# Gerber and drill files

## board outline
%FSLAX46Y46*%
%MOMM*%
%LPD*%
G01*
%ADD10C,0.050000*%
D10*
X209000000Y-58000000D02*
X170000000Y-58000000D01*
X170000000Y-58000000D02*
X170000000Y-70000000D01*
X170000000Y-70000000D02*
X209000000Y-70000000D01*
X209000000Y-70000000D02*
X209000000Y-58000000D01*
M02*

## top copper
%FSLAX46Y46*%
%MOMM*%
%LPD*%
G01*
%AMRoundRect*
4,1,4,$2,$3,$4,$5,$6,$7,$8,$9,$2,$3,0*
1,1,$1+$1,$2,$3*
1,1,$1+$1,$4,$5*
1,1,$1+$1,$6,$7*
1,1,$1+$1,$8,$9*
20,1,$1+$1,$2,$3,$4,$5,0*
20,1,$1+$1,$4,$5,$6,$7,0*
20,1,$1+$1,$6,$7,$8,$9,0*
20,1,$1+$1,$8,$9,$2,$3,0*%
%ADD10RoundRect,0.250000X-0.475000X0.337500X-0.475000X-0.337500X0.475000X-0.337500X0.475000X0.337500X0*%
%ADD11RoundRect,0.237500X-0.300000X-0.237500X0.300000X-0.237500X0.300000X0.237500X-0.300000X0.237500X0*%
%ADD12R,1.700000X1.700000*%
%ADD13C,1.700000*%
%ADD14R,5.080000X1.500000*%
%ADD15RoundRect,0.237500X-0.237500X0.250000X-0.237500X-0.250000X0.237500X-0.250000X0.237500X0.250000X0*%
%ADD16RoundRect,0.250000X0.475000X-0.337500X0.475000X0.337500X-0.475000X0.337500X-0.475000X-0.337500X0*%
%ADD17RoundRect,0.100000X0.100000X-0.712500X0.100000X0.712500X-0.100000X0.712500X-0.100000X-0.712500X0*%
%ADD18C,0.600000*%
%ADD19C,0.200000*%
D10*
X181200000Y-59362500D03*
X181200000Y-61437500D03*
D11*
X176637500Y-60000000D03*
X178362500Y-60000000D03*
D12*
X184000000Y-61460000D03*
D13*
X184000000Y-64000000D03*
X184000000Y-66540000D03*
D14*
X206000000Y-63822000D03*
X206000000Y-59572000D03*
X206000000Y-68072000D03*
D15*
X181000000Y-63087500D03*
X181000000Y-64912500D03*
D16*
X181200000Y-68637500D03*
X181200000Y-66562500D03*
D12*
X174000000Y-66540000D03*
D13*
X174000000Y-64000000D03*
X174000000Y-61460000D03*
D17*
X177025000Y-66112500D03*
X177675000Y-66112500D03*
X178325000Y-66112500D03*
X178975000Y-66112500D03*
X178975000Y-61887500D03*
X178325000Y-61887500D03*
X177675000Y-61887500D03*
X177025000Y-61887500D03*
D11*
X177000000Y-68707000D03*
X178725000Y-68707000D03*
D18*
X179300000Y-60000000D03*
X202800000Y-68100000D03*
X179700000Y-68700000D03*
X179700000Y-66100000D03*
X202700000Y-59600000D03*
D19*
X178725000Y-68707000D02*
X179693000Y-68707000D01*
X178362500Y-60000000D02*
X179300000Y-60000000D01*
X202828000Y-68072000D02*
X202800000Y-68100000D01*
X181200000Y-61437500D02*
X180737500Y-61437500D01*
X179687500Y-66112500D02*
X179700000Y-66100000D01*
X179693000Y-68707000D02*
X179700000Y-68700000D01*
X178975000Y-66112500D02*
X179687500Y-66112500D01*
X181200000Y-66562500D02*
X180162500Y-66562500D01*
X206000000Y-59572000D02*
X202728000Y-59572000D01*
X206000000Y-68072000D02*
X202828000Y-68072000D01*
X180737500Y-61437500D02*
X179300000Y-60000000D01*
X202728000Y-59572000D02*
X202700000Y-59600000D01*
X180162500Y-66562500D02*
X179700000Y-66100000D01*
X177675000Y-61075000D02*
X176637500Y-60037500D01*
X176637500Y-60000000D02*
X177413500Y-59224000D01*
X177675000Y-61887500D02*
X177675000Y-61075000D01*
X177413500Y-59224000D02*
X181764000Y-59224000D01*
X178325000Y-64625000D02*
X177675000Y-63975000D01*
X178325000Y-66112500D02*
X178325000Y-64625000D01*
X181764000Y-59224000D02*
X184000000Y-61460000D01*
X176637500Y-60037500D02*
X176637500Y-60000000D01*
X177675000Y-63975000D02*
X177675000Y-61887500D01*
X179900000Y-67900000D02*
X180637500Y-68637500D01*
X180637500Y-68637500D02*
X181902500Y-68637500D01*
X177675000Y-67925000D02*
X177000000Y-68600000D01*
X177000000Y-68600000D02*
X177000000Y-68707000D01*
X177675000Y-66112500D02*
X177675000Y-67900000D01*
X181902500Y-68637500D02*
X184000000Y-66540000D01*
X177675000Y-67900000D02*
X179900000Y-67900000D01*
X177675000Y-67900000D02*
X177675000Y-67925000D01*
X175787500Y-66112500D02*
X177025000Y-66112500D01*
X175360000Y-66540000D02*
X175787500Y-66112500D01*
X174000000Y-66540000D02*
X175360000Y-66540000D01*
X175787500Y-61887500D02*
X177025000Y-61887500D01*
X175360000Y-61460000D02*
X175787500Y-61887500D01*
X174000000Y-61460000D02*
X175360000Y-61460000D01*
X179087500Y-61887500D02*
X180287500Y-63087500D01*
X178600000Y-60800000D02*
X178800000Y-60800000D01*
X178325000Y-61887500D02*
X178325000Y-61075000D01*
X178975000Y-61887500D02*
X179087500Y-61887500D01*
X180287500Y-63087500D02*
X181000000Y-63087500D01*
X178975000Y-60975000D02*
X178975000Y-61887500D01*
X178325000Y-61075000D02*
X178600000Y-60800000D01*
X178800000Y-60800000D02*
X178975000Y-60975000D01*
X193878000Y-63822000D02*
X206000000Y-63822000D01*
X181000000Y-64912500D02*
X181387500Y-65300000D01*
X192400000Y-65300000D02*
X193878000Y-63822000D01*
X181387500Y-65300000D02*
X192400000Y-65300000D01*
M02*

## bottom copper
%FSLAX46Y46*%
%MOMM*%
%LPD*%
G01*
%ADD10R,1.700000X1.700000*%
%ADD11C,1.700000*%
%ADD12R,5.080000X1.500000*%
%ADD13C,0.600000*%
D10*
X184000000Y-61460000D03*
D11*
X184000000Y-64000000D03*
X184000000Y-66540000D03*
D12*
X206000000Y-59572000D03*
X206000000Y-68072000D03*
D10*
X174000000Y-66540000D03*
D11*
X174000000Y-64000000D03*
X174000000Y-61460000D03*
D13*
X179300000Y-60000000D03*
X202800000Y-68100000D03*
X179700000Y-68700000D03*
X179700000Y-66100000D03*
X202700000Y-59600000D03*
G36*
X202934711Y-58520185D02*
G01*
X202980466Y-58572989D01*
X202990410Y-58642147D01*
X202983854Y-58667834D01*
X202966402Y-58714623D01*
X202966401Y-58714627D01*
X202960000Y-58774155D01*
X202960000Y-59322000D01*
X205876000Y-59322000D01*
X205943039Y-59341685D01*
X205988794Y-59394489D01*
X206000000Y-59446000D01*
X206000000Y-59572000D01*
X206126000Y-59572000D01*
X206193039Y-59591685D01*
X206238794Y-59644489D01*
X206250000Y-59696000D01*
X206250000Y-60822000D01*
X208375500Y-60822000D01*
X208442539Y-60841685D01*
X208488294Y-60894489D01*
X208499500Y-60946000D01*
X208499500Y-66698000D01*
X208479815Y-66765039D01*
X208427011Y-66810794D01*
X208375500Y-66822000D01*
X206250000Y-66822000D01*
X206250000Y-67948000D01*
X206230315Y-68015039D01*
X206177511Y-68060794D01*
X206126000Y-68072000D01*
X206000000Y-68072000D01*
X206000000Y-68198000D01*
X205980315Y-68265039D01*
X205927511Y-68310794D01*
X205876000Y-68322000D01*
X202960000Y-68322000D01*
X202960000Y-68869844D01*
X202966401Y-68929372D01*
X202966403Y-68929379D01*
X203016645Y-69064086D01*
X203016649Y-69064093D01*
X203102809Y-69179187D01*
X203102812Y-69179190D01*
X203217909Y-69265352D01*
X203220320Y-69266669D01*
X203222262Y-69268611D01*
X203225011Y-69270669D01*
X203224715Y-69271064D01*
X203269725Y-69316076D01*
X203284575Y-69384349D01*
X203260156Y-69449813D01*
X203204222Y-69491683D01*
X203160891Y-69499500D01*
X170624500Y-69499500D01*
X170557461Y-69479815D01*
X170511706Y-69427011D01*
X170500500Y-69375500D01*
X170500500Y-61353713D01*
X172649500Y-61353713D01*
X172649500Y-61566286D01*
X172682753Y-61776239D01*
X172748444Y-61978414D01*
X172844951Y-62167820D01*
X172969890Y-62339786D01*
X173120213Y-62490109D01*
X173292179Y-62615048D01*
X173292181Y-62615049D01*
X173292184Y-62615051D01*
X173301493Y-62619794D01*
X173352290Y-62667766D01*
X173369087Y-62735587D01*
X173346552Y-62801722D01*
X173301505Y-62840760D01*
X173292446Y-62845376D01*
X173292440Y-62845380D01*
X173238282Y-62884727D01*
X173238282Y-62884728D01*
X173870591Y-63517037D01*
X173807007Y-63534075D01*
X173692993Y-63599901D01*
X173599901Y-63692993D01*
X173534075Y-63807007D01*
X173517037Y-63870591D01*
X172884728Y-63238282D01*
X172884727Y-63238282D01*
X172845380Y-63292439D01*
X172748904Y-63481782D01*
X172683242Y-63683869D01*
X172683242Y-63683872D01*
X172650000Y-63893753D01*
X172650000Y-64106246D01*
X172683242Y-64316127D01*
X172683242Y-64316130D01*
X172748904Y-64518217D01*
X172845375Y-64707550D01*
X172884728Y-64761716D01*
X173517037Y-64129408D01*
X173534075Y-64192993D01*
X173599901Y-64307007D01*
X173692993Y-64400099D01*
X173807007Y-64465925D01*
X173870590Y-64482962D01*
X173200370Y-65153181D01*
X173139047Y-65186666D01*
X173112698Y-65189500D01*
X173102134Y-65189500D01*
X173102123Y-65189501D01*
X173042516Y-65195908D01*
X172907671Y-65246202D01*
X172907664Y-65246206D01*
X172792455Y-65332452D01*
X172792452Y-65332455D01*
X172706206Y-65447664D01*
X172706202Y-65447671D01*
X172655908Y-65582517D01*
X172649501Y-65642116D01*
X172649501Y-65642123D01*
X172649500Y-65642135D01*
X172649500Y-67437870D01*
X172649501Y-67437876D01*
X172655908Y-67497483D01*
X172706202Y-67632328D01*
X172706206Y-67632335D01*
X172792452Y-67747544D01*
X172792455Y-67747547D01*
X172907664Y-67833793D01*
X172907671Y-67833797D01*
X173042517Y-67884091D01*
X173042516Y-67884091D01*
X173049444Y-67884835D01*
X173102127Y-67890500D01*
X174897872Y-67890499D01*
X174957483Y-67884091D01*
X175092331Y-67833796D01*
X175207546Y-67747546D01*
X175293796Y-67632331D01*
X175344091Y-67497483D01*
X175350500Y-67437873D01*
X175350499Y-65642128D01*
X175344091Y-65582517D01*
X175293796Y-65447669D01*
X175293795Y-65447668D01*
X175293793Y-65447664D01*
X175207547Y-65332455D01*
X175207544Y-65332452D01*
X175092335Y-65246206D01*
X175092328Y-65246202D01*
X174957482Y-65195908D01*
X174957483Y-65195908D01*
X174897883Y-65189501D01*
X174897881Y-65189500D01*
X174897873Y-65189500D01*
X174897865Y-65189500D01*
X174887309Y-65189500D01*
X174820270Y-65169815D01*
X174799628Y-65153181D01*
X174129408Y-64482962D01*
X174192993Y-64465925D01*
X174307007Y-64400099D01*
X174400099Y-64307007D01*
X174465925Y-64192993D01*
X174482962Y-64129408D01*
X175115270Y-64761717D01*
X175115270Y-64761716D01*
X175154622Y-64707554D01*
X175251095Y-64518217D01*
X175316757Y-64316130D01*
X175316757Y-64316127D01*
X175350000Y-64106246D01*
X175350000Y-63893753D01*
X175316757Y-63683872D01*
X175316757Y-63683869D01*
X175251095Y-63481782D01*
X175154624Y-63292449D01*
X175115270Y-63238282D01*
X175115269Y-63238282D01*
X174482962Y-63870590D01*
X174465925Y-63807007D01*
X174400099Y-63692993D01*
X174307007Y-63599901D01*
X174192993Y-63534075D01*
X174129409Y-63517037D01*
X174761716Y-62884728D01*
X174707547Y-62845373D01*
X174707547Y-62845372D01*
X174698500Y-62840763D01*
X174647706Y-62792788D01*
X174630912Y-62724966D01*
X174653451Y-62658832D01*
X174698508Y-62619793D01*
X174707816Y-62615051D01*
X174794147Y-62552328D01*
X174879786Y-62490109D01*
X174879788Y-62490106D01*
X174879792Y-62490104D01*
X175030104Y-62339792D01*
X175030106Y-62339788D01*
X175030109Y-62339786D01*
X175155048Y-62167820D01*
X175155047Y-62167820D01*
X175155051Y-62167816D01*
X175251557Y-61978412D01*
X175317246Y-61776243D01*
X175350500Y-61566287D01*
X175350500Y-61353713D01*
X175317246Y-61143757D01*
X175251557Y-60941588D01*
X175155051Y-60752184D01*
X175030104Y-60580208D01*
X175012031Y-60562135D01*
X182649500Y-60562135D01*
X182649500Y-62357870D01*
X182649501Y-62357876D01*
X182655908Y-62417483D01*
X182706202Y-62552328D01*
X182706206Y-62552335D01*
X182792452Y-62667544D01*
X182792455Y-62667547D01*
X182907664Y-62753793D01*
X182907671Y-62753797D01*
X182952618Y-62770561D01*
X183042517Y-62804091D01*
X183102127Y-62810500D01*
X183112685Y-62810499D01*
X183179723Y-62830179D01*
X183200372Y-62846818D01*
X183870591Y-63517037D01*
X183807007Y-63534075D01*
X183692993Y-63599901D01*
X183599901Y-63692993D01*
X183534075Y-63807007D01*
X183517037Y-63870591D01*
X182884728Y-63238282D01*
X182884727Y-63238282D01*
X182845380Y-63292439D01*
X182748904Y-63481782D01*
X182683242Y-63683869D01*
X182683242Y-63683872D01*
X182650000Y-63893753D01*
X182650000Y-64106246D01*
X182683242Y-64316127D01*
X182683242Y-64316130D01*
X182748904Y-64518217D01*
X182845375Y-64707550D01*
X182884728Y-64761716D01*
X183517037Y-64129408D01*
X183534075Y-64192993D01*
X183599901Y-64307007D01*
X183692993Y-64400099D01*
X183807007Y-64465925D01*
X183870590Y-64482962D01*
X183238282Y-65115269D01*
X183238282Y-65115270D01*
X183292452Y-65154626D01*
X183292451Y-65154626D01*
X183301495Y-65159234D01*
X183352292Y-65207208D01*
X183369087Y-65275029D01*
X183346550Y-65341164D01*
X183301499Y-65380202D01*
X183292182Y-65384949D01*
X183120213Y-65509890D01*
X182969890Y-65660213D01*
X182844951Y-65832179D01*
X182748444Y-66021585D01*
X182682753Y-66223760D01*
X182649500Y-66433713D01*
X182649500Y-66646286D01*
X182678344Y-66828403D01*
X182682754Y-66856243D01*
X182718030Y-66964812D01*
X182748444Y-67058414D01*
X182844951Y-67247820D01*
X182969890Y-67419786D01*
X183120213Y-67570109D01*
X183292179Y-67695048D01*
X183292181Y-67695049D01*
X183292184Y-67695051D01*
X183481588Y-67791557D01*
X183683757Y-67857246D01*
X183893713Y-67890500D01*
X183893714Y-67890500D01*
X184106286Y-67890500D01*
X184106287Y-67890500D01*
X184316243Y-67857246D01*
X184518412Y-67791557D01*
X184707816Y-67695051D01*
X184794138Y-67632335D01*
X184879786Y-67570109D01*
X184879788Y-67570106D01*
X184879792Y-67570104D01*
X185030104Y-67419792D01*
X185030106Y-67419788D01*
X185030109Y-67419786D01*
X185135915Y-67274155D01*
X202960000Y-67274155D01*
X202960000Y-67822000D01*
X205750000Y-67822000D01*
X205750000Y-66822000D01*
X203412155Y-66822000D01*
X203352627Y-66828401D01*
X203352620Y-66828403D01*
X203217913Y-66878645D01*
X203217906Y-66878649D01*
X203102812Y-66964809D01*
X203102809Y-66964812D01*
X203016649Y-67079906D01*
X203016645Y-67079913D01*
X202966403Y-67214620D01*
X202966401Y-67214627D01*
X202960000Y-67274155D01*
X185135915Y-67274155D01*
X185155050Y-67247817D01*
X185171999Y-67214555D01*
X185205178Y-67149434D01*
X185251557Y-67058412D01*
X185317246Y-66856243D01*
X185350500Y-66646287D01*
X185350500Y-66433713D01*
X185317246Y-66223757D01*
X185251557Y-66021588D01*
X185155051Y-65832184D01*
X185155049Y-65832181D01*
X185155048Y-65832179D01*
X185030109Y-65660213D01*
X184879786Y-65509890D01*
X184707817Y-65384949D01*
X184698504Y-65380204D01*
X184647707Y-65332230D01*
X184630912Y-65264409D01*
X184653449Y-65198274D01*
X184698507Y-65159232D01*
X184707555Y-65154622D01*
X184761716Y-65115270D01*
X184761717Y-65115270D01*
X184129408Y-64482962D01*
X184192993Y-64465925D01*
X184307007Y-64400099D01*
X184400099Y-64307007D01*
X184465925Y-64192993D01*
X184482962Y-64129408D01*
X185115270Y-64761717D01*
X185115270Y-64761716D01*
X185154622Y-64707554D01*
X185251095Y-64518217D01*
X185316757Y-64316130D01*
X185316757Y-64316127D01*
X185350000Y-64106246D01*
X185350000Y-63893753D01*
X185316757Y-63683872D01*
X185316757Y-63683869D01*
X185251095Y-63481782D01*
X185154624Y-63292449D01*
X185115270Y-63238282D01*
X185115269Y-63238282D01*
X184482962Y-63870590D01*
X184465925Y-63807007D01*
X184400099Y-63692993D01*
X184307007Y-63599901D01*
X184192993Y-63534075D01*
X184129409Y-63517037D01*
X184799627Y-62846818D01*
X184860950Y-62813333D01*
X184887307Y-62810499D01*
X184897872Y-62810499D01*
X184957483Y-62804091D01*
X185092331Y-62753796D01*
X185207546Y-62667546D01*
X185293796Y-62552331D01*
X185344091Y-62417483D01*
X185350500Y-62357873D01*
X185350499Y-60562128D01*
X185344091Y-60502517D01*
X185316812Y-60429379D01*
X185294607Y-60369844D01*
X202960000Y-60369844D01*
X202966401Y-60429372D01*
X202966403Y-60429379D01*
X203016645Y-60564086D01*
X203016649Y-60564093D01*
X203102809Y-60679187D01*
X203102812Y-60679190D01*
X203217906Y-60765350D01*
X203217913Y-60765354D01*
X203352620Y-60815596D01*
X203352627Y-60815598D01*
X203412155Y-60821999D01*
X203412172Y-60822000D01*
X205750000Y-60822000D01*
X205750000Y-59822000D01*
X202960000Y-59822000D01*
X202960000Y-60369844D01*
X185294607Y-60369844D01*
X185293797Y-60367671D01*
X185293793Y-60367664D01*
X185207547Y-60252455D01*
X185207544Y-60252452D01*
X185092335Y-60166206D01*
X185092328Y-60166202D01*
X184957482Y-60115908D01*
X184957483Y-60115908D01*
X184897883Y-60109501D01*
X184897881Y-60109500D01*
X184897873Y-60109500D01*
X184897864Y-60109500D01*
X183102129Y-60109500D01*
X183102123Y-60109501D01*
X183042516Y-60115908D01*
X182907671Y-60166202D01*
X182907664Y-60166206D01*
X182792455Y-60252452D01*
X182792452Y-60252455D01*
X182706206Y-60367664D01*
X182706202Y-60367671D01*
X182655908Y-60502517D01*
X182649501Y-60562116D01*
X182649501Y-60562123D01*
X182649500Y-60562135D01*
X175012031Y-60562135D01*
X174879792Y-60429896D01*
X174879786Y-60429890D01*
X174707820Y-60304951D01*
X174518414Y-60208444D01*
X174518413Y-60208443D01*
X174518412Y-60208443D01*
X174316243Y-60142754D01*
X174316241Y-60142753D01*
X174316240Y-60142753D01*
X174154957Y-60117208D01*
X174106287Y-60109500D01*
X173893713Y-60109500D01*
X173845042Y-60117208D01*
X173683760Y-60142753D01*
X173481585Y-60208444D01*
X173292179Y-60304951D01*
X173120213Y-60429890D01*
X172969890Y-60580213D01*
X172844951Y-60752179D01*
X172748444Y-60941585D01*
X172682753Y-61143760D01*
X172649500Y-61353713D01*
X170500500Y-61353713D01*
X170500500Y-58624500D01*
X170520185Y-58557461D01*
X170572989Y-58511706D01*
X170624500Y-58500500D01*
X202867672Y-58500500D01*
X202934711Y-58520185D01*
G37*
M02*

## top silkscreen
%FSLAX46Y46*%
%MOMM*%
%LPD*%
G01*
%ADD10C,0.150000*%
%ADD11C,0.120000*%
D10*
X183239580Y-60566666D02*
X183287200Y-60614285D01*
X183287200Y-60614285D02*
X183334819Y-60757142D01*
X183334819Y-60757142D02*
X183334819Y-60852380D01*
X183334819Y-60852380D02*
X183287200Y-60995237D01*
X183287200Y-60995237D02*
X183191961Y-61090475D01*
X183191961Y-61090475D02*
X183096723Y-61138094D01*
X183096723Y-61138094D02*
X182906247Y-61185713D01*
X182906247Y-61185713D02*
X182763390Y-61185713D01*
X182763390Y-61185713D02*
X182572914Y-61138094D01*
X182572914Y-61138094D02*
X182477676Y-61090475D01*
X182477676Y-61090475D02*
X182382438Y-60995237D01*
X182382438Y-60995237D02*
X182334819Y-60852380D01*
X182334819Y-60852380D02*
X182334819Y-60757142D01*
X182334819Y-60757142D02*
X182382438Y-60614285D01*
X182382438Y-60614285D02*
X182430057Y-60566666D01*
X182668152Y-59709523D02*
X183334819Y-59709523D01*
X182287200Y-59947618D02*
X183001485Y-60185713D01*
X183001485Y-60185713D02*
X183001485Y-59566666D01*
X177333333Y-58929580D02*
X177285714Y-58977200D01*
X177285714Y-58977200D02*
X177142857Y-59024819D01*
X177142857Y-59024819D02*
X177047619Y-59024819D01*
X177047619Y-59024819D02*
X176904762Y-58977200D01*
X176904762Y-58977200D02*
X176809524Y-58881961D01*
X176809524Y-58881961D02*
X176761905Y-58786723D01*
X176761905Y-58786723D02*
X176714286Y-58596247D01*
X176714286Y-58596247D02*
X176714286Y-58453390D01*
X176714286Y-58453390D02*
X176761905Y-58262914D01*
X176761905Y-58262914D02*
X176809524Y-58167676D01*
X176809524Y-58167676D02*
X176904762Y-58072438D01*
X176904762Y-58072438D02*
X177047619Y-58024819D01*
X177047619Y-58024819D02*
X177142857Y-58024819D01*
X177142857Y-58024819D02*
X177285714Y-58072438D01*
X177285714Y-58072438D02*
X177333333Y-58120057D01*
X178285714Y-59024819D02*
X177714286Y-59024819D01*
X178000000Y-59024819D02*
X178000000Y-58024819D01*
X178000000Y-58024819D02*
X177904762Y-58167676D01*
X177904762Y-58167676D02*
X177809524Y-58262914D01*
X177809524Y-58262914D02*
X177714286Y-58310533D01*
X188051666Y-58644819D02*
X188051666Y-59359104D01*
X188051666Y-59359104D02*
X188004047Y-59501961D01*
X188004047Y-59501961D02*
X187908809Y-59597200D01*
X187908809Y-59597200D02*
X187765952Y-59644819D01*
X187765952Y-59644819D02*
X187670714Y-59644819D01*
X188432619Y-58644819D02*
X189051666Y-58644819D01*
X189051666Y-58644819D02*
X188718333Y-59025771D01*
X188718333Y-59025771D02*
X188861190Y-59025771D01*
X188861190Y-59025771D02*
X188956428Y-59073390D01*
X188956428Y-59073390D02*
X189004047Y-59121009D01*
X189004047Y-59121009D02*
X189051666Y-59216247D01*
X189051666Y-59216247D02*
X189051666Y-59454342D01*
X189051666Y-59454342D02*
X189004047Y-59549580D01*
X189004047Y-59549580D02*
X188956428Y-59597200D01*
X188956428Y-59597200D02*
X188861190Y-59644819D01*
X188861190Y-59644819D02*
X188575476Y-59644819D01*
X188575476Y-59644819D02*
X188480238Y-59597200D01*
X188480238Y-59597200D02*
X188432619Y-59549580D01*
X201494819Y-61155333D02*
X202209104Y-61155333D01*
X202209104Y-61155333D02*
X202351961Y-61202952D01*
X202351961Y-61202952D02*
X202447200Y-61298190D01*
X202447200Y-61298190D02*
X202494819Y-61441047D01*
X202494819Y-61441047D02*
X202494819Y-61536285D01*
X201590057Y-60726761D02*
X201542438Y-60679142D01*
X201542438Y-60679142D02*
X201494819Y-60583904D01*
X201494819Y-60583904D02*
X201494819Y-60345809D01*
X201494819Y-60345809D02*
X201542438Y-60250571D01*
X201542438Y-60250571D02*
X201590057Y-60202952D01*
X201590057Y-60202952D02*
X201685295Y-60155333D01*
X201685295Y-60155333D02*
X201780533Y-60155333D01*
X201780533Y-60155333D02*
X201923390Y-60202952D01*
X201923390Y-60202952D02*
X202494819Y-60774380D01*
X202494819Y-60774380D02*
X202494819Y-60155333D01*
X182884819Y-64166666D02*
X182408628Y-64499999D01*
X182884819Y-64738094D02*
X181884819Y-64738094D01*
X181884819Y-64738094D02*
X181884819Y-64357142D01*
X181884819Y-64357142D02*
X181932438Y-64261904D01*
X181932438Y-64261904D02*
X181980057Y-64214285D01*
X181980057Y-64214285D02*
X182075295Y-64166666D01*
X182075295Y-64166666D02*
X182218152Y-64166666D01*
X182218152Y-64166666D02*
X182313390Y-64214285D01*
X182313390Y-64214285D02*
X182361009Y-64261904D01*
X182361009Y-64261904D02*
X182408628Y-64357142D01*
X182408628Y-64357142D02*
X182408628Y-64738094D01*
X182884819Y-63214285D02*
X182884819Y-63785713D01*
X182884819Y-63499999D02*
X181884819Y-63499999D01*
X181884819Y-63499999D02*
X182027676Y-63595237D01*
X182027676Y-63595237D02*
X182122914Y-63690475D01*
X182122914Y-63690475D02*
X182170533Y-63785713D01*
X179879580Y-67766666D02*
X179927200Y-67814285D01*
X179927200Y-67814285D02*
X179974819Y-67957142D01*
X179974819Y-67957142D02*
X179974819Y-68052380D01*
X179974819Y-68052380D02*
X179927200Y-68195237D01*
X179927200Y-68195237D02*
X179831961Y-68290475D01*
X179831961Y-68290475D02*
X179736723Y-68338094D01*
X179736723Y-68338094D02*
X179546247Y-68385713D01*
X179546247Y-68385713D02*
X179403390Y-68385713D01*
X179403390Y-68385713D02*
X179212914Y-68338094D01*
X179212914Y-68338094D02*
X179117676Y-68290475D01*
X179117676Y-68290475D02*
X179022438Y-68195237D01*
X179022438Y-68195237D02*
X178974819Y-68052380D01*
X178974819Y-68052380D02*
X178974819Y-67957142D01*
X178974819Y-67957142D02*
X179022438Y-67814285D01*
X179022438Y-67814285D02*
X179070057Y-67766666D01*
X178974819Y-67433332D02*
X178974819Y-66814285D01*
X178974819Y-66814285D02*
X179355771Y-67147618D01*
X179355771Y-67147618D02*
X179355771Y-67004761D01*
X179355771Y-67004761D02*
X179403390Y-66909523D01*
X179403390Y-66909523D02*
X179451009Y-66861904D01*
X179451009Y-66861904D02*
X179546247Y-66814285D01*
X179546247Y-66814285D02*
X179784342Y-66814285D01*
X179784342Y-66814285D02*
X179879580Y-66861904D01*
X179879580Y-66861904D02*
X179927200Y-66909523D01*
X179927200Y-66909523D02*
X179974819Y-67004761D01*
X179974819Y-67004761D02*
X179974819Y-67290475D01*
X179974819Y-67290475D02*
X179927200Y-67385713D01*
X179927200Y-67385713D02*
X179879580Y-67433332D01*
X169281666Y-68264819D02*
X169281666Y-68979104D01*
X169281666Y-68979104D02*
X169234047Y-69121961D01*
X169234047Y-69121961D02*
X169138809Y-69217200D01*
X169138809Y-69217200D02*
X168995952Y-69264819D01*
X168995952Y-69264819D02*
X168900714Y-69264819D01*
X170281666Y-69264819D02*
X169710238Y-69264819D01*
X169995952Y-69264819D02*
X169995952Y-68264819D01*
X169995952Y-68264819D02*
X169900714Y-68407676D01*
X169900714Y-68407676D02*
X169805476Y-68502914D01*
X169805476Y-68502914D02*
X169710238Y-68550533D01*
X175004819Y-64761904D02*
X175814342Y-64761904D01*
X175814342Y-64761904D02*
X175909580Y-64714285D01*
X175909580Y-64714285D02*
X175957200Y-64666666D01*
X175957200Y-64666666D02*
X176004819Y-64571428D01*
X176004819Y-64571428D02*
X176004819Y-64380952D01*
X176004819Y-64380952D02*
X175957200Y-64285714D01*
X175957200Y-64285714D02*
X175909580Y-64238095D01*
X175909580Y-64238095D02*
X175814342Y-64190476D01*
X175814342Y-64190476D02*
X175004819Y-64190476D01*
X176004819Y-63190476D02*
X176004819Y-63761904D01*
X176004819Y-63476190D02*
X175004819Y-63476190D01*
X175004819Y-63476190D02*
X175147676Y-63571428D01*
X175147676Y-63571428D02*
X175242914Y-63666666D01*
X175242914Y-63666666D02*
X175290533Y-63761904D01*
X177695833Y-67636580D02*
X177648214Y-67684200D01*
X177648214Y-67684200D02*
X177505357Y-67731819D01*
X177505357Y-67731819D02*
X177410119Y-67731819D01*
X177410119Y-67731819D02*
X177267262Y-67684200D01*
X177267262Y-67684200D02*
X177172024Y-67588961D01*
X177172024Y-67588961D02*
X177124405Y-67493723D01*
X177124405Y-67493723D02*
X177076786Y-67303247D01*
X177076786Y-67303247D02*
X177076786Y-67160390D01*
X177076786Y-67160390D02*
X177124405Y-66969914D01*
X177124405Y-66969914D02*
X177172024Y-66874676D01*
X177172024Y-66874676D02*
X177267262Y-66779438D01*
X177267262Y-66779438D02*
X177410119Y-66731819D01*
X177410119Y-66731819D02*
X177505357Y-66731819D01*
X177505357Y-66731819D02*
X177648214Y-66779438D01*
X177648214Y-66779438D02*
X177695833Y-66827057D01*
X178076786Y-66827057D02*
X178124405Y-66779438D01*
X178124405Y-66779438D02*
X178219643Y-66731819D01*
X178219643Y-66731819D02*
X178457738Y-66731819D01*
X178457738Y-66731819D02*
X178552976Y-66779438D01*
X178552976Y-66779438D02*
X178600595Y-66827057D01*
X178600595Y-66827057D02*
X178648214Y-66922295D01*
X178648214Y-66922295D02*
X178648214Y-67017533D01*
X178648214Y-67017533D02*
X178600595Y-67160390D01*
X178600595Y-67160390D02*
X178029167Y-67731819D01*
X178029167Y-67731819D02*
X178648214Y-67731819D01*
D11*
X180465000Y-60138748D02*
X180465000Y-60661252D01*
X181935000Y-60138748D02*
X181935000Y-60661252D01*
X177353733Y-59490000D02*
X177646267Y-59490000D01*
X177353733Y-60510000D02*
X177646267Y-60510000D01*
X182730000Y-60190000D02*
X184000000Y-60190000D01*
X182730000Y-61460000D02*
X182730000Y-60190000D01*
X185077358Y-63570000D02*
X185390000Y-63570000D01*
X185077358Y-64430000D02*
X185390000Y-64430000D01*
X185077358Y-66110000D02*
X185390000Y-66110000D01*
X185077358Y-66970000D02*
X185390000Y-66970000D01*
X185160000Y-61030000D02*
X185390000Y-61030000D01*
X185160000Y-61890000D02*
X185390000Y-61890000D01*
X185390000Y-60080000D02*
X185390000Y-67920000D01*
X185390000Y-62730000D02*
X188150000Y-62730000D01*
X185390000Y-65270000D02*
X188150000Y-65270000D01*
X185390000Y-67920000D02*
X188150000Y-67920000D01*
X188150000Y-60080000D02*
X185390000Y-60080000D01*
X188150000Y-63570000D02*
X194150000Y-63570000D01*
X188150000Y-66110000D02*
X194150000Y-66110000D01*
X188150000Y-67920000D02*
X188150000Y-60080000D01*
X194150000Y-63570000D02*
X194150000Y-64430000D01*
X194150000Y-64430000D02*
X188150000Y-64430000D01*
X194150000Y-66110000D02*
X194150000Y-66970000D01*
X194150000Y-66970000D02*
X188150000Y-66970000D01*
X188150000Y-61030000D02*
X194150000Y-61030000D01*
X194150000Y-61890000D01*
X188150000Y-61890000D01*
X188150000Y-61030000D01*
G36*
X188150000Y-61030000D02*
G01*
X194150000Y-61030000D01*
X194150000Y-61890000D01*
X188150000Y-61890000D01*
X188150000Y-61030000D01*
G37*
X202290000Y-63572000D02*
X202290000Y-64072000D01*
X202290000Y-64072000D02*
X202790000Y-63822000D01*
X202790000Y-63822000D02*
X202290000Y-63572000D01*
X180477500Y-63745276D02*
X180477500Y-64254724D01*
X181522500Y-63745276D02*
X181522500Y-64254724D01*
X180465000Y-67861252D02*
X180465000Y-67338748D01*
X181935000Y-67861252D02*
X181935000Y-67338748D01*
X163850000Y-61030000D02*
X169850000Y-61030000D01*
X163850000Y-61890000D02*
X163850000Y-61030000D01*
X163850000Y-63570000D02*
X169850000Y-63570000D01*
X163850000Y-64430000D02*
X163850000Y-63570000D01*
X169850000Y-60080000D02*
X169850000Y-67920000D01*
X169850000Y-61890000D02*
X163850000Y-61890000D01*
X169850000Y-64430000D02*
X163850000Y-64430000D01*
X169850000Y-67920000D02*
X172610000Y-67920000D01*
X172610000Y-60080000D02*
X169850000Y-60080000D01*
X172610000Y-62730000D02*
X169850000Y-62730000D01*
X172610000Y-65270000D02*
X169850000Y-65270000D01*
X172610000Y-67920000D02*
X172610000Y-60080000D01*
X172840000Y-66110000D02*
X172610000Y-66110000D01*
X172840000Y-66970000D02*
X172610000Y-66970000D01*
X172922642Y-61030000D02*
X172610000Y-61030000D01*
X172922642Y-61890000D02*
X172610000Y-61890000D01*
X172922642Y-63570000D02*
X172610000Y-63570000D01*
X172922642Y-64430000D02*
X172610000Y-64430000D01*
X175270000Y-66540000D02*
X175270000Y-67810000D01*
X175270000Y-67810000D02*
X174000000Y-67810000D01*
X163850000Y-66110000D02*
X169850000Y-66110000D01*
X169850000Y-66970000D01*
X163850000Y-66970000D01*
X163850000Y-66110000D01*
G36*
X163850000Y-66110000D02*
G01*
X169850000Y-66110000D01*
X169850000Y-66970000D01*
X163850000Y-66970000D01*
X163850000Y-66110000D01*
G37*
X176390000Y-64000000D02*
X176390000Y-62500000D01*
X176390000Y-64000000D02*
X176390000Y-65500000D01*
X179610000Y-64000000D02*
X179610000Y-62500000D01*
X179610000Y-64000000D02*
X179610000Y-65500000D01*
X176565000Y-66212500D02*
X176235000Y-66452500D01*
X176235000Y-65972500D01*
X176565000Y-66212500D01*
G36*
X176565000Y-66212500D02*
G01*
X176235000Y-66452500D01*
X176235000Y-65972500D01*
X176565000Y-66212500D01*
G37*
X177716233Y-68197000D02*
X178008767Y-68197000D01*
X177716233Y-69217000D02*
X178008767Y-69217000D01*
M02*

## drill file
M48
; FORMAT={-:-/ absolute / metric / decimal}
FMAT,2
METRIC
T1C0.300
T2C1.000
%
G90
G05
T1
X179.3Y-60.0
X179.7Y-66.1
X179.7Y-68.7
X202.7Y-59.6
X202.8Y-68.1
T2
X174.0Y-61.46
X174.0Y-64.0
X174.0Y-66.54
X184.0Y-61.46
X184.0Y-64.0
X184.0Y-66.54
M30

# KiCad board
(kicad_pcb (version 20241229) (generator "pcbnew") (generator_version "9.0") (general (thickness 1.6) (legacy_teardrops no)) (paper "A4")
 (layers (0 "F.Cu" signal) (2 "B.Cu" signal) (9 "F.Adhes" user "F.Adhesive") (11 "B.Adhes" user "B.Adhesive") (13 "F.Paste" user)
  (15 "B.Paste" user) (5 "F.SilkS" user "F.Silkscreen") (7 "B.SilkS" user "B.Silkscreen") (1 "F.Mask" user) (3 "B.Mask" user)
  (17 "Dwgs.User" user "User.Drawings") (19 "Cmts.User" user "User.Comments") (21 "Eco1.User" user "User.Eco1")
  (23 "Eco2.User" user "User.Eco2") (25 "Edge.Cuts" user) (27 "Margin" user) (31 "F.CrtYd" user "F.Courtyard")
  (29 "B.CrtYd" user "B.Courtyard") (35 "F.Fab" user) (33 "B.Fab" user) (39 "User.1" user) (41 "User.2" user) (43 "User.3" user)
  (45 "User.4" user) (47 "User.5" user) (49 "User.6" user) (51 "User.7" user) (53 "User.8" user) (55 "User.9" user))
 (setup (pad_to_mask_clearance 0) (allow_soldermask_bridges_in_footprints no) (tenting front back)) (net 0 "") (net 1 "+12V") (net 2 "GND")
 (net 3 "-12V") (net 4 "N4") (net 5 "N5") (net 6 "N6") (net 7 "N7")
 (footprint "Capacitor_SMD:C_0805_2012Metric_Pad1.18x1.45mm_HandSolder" (layer "F.Cu") (at 181.2 60.4 -90)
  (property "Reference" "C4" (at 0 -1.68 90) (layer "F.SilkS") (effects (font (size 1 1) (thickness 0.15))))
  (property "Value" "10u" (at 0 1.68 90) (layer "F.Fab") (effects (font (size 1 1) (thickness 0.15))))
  (fp_line (start -0.261252 0.735) (end 0.261252 0.735) (stroke (width 0.12) (type solid)) (layer "F.SilkS"))
  (fp_line (start -0.261252 -0.735) (end 0.261252 -0.735) (stroke (width 0.12) (type solid)) (layer "F.SilkS"))
  (pad "1" smd roundrect (at -1.0375 0 270) (size 1.175 1.45) (layers "F.Cu" "F.Mask" "F.Paste") (roundrect_rratio 0.212766) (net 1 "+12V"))
  (pad "2" smd roundrect (at 1.0375 0 270) (size 1.175 1.45) (layers "F.Cu" "F.Mask" "F.Paste") (roundrect_rratio 0.212766) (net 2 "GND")))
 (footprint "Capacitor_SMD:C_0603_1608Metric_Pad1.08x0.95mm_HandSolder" (layer "F.Cu") (at 177.5 60)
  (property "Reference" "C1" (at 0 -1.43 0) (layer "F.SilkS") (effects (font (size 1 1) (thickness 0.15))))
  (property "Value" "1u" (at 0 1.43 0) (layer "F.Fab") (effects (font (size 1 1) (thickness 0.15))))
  (fp_line (start -0.146267 -0.51) (end 0.146267 -0.51) (stroke (width 0.12) (type solid)) (layer "F.SilkS"))
  (fp_line (start -0.146267 0.51) (end 0.146267 0.51) (stroke (width 0.12) (type solid)) (layer "F.SilkS"))
  (pad "1" smd roundrect (at -0.8625 0) (size 1.075 0.95) (layers "F.Cu" "F.Mask" "F.Paste") (roundrect_rratio 0.25) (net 1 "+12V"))
  (pad "2" smd roundrect (at 0.8625 0) (size 1.075 0.95) (layers "F.Cu" "F.Mask" "F.Paste") (roundrect_rratio 0.25) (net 2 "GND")))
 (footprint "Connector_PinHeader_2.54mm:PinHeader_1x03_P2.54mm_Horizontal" (layer "F.Cu") (at 184 61.46)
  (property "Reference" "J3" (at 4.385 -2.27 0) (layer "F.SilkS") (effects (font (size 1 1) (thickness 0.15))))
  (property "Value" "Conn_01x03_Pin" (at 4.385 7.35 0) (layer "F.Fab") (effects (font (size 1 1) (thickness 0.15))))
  (fp_line (start -1.27 -1.27) (end 0 -1.27) (stroke (width 0.12) (type solid)) (layer "F.SilkS"))
  (fp_line (start -1.27 0) (end -1.27 -1.27) (stroke (width 0.12) (type solid)) (layer "F.SilkS"))
  (fp_line (start 1.077358 2.11) (end 1.39 2.11) (stroke (width 0.12) (type solid)) (layer "F.SilkS"))
  (fp_line (start 1.077358 2.97) (end 1.39 2.97) (stroke (width 0.12) (type solid)) (layer "F.SilkS"))
  (fp_line (start 1.077358 4.65) (end 1.39 4.65) (stroke (width 0.12) (type solid)) (layer "F.SilkS"))
  (fp_line (start 1.077358 5.51) (end 1.39 5.51) (stroke (width 0.12) (type solid)) (layer "F.SilkS"))
  (fp_line (start 1.16 -0.43) (end 1.39 -0.43) (stroke (width 0.12) (type solid)) (layer "F.SilkS"))
  (fp_line (start 1.16 0.43) (end 1.39 0.43) (stroke (width 0.12) (type solid)) (layer "F.SilkS"))
  (fp_line (start 1.39 -1.38) (end 1.39 6.46) (stroke (width 0.12) (type solid)) (layer "F.SilkS"))
  (fp_line (start 1.39 1.27) (end 4.15 1.27) (stroke (width 0.12) (type solid)) (layer "F.SilkS"))
  (fp_line (start 1.39 3.81) (end 4.15 3.81) (stroke (width 0.12) (type solid)) (layer "F.SilkS"))
  (fp_line (start 1.39 6.46) (end 4.15 6.46) (stroke (width 0.12) (type solid)) (layer "F.SilkS"))
  (fp_line (start 4.15 -1.38) (end 1.39 -1.38) (stroke (width 0.12) (type solid)) (layer "F.SilkS"))
  (fp_line (start 4.15 2.11) (end 10.15 2.11) (stroke (width 0.12) (type solid)) (layer "F.SilkS"))
  (fp_line (start 4.15 4.65) (end 10.15 4.65) (stroke (width 0.12) (type solid)) (layer "F.SilkS"))
  (fp_line (start 4.15 6.46) (end 4.15 -1.38) (stroke (width 0.12) (type solid)) (layer "F.SilkS"))
  (fp_line (start 10.15 2.11) (end 10.15 2.97) (stroke (width 0.12) (type solid)) (layer "F.SilkS"))
  (fp_line (start 10.15 2.97) (end 4.15 2.97) (stroke (width 0.12) (type solid)) (layer "F.SilkS"))
  (fp_line (start 10.15 4.65) (end 10.15 5.51) (stroke (width 0.12) (type solid)) (layer "F.SilkS"))
  (fp_line (start 10.15 5.51) (end 4.15 5.51) (stroke (width 0.12) (type solid)) (layer "F.SilkS"))
  (fp_rect (start 4.15 -0.43) (end 10.15 0.43) (stroke (width 0.12) (type solid)) (fill yes) (layer "F.SilkS"))
  (pad "1" thru_hole rect (at 0 0) (size 1.7 1.7) (drill 1) (layers "*.Cu" "*.Mask") (remove_unused_layers no) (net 1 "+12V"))
  (pad "2" thru_hole circle (at 0 2.54) (size 1.7 1.7) (drill 1) (layers "*.Cu" "*.Mask") (remove_unused_layers no) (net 2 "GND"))
  (pad "3" thru_hole circle (at 0 5.08) (size 1.7 1.7) (drill 1) (layers "*.Cu" "*.Mask") (remove_unused_layers no) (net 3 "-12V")))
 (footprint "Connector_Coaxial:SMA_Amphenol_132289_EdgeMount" (layer "F.Cu") (at 206 63.822)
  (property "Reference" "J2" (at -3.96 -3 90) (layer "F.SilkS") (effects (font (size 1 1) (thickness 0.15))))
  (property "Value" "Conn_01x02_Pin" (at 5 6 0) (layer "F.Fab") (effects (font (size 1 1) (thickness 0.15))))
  (fp_line (start -3.71 -0.25) (end -3.71 0.25) (stroke (width 0.12) (type solid)) (layer "F.SilkS"))
  (fp_line (start -3.71 0.25) (end -3.21 0) (stroke (width 0.12) (type solid)) (layer "F.SilkS"))
  (fp_line (start -3.21 0) (end -3.71 -0.25) (stroke (width 0.12) (type solid)) (layer "F.SilkS"))
  (pad "1" smd rect (at 0 0 90) (size 1.5 5.08) (layers "F.Cu" "F.Mask" "F.Paste") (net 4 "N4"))
  (pad "2" smd rect (at 0 -4.25 90) (size 1.5 5.08) (layers "F.Cu" "F.Mask" "F.Paste") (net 2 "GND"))
  (pad "2" smd rect (at 0 -4.25 90) (size 1.5 5.08) (layers "B.Cu" "B.Mask" "B.Paste") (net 2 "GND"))
  (pad "2" smd rect (at 0 4.25 90) (size 1.5 5.08) (layers "F.Cu" "F.Mask" "F.Paste") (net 2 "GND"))
  (pad "2" smd rect (at 0 4.25 90) (size 1.5 5.08) (layers "B.Cu" "B.Mask" "B.Paste") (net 2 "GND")))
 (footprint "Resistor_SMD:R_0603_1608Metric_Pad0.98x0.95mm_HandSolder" (layer "F.Cu") (at 181 64 -90)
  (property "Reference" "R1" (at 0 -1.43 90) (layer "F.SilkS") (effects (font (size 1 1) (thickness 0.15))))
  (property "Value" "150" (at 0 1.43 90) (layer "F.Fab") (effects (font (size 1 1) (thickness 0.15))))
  (fp_line (start -0.254724 0.5225) (end 0.254724 0.5225) (stroke (width 0.12) (type solid)) (layer "F.SilkS"))
  (fp_line (start -0.254724 -0.5225) (end 0.254724 -0.5225) (stroke (width 0.12) (type solid)) (layer "F.SilkS"))
  (pad "1" smd roundrect (at -0.9125 0 270) (size 0.975 0.95) (layers "F.Cu" "F.Mask" "F.Paste") (roundrect_rratio 0.25) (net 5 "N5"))
  (pad "2" smd roundrect (at 0.9125 0 270) (size 0.975 0.95) (layers "F.Cu" "F.Mask" "F.Paste") (roundrect_rratio 0.25) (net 4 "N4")))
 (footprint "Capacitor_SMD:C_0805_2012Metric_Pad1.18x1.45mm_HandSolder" (layer "F.Cu") (at 181.2 67.6 90)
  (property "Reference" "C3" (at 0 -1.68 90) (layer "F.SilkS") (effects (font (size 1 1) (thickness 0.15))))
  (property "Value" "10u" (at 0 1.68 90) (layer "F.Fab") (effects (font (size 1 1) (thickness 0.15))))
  (fp_line (start -0.261252 -0.735) (end 0.261252 -0.735) (stroke (width 0.12) (type solid)) (layer "F.SilkS"))
  (fp_line (start -0.261252 0.735) (end 0.261252 0.735) (stroke (width 0.12) (type solid)) (layer "F.SilkS"))
  (pad "1" smd roundrect (at -1.0375 0 90) (size 1.175 1.45) (layers "F.Cu" "F.Mask" "F.Paste") (roundrect_rratio 0.212766) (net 3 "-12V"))
  (pad "2" smd roundrect (at 1.0375 0 90) (size 1.175 1.45) (layers "F.Cu" "F.Mask" "F.Paste") (roundrect_rratio 0.212766) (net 2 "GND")))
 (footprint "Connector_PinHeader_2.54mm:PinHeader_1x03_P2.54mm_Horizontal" (layer "F.Cu") (at 174 66.54 180)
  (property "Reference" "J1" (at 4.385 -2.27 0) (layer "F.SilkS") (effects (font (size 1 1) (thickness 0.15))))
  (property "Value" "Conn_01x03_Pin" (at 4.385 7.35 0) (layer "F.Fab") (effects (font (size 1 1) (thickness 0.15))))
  (fp_line (start 10.15 5.51) (end 4.15 5.51) (stroke (width 0.12) (type solid)) (layer "F.SilkS"))
  (fp_line (start 10.15 4.65) (end 10.15 5.51) (stroke (width 0.12) (type solid)) (layer "F.SilkS"))
  (fp_line (start 10.15 2.97) (end 4.15 2.97) (stroke (width 0.12) (type solid)) (layer "F.SilkS"))
  (fp_line (start 10.15 2.11) (end 10.15 2.97) (stroke (width 0.12) (type solid)) (layer "F.SilkS"))
  (fp_line (start 4.15 6.46) (end 4.15 -1.38) (stroke (width 0.12) (type solid)) (layer "F.SilkS"))
  (fp_line (start 4.15 4.65) (end 10.15 4.65) (stroke (width 0.12) (type solid)) (layer "F.SilkS"))
  (fp_line (start 4.15 2.11) (end 10.15 2.11) (stroke (width 0.12) (type solid)) (layer "F.SilkS"))
  (fp_line (start 4.15 -1.38) (end 1.39 -1.38) (stroke (width 0.12) (type solid)) (layer "F.SilkS"))
  (fp_line (start 1.39 6.46) (end 4.15 6.46) (stroke (width 0.12) (type solid)) (layer "F.SilkS"))
  (fp_line (start 1.39 3.81) (end 4.15 3.81) (stroke (width 0.12) (type solid)) (layer "F.SilkS"))
  (fp_line (start 1.39 1.27) (end 4.15 1.27) (stroke (width 0.12) (type solid)) (layer "F.SilkS"))
  (fp_line (start 1.39 -1.38) (end 1.39 6.46) (stroke (width 0.12) (type solid)) (layer "F.SilkS"))
  (fp_line (start 1.16 0.43) (end 1.39 0.43) (stroke (width 0.12) (type solid)) (layer "F.SilkS"))
  (fp_line (start 1.16 -0.43) (end 1.39 -0.43) (stroke (width 0.12) (type solid)) (layer "F.SilkS"))
  (fp_line (start 1.077358 5.51) (end 1.39 5.51) (stroke (width 0.12) (type solid)) (layer "F.SilkS"))
  (fp_line (start 1.077358 4.65) (end 1.39 4.65) (stroke (width 0.12) (type solid)) (layer "F.SilkS"))
  (fp_line (start 1.077358 2.97) (end 1.39 2.97) (stroke (width 0.12) (type solid)) (layer "F.SilkS"))
  (fp_line (start 1.077358 2.11) (end 1.39 2.11) (stroke (width 0.12) (type solid)) (layer "F.SilkS"))
  (fp_line (start -1.27 0) (end -1.27 -1.27) (stroke (width 0.12) (type solid)) (layer "F.SilkS"))
  (fp_line (start -1.27 -1.27) (end 0 -1.27) (stroke (width 0.12) (type solid)) (layer "F.SilkS"))
  (fp_rect (start 4.15 -0.43) (end 10.15 0.43) (stroke (width 0.12) (type solid)) (fill yes) (layer "F.SilkS"))
  (pad "1" thru_hole rect (at 0 0 180) (size 1.7 1.7) (drill 1) (layers "*.Cu" "*.Mask") (remove_unused_layers no) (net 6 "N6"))
  (pad "2" thru_hole circle (at 0 2.54 180) (size 1.7 1.7) (drill 1) (layers "*.Cu" "*.Mask") (remove_unused_layers no) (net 2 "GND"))
  (pad "3" thru_hole circle (at 0 5.08 180) (size 1.7 1.7) (drill 1) (layers "*.Cu" "*.Mask") (remove_unused_layers no) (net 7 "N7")))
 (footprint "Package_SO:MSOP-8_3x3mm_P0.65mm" (layer "F.Cu") (at 178 64 90)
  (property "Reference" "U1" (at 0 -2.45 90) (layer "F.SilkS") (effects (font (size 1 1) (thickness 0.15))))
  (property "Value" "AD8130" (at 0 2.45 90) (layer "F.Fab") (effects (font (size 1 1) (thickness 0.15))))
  (fp_line (start 0 -1.61) (end 1.5 -1.61) (stroke (width 0.12) (type solid)) (layer "F.SilkS"))
  (fp_line (start 0 -1.61) (end -1.5 -1.61) (stroke (width 0.12) (type solid)) (layer "F.SilkS"))
  (fp_line (start 0 1.61) (end 1.5 1.61) (stroke (width 0.12) (type solid)) (layer "F.SilkS"))
  (fp_line (start 0 1.61) (end -1.5 1.61) (stroke (width 0.12) (type solid)) (layer "F.SilkS"))
  (fp_poly
   (pts (xy -2.2125 -1.435) (xy -2.4525 -1.765) (xy -1.9725 -1.765)) (stroke (width 0.12) (type solid)) (fill yes) (layer "F.SilkS"))
  (pad "1" smd roundrect (at -2.1125 -0.975 90) (size 1.625 0.4) (layers "F.Cu" "F.Mask" "F.Paste") (roundrect_rratio 0.25) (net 6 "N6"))
  (pad "2" smd roundrect (at -2.1125 -0.325 90) (size 1.625 0.4) (layers "F.Cu" "F.Mask" "F.Paste") (roundrect_rratio 0.25) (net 3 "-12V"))
  (pad "3" smd roundrect (at -2.1125 0.325 90) (size 1.625 0.4) (layers "F.Cu" "F.Mask" "F.Paste") (roundrect_rratio 0.25) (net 1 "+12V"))
  (pad "4" smd roundrect (at -2.1125 0.975 90) (size 1.625 0.4) (layers "F.Cu" "F.Mask" "F.Paste") (roundrect_rratio 0.25) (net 2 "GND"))
  (pad "5" smd roundrect (at 2.1125 0.975 90) (size 1.625 0.4) (layers "F.Cu" "F.Mask" "F.Paste") (roundrect_rratio 0.25) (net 5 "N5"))
  (pad "6" smd roundrect (at 2.1125 0.325 90) (size 1.625 0.4) (layers "F.Cu" "F.Mask" "F.Paste") (roundrect_rratio 0.25) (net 5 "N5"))
  (pad "7" smd roundrect (at 2.1125 -0.325 90) (size 1.625 0.4) (layers "F.Cu" "F.Mask" "F.Paste") (roundrect_rratio 0.25) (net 1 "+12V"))
  (pad "8" smd roundrect (at 2.1125 -0.975 90) (size 1.625 0.4) (layers "F.Cu" "F.Mask" "F.Paste") (roundrect_rratio 0.25) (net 7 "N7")))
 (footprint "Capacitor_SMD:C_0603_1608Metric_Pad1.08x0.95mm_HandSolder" (layer "F.Cu") (at 177.8625 68.707)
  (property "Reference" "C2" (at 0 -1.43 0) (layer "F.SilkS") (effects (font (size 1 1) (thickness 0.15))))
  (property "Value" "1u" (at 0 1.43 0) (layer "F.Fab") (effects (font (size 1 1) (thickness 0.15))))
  (fp_line (start -0.146267 -0.51) (end 0.146267 -0.51) (stroke (width 0.12) (type solid)) (layer "F.SilkS"))
  (fp_line (start -0.146267 0.51) (end 0.146267 0.51) (stroke (width 0.12) (type solid)) (layer "F.SilkS"))
  (pad "1" smd roundrect (at -0.8625 0) (size 1.075 0.95) (layers "F.Cu" "F.Mask" "F.Paste") (roundrect_rratio 0.25) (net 3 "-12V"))
  (pad "2" smd roundrect (at 0.8625 0) (size 1.075 0.95) (layers "F.Cu" "F.Mask" "F.Paste") (roundrect_rratio 0.25) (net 2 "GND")))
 (gr_line (start 209 58) (end 170 58) (stroke (width 0.05) (type default)) (layer "Edge.Cuts"))
 (gr_line (start 170 58) (end 170 70) (stroke (width 0.05) (type default)) (layer "Edge.Cuts"))
 (gr_line (start 170 70) (end 209 70) (stroke (width 0.05) (type default)) (layer "Edge.Cuts"))
 (gr_line (start 209 70) (end 209 58) (stroke (width 0.05) (type default)) (layer "Edge.Cuts"))
 (segment (start 178.725 68.707) (end 179.693 68.707) (width 0.2) (layer "F.Cu") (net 2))
 (segment (start 178.3625 60) (end 179.3 60) (width 0.2) (layer "F.Cu") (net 2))
 (segment (start 202.828 68.072) (end 202.8 68.1) (width 0.2) (layer "F.Cu") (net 2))
 (segment (start 181.2 61.4375) (end 180.7375 61.4375) (width 0.2) (layer "F.Cu") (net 2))
 (segment (start 179.6875 66.1125) (end 179.7 66.1) (width 0.2) (layer "F.Cu") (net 2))
 (segment (start 179.693 68.707) (end 179.7 68.7) (width 0.2) (layer "F.Cu") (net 2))
 (segment (start 178.975 66.1125) (end 179.6875 66.1125) (width 0.2) (layer "F.Cu") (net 2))
 (segment (start 181.2 66.5625) (end 180.1625 66.5625) (width 0.2) (layer "F.Cu") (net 2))
 (segment (start 206 59.572) (end 202.728 59.572) (width 0.2) (layer "F.Cu") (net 2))
 (segment (start 206 68.072) (end 202.828 68.072) (width 0.2) (layer "F.Cu") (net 2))
 (segment (start 180.7375 61.4375) (end 179.3 60) (width 0.2) (layer "F.Cu") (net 2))
 (segment (start 202.728 59.572) (end 202.7 59.6) (width 0.2) (layer "F.Cu") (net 2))
 (segment (start 180.1625 66.5625) (end 179.7 66.1) (width 0.2) (layer "F.Cu") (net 2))
 (via (at 179.3 60) (size 0.6) (drill 0.3) (layers "F.Cu" "B.Cu") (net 2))
 (via (at 202.8 68.1) (size 0.6) (drill 0.3) (layers "F.Cu" "B.Cu") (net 2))
 (via (at 179.7 68.7) (size 0.6) (drill 0.3) (layers "F.Cu" "B.Cu") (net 2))
 (via (at 179.7 66.1) (size 0.6) (drill 0.3) (layers "F.Cu" "B.Cu") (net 2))
 (via (at 202.7 59.6) (size 0.6) (drill 0.3) (layers "F.Cu" "B.Cu") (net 2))
 (segment (start 177.675 61.075) (end 176.6375 60.0375) (width 0.2) (layer "F.Cu") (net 1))
 (segment (start 176.6375 60) (end 177.4135 59.224) (width 0.2) (layer "F.Cu") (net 1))
 (segment (start 177.675 61.8875) (end 177.675 61.075) (width 0.2) (layer "F.Cu") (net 1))
 (segment (start 177.4135 59.224) (end 181.764 59.224) (width 0.2) (layer "F.Cu") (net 1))
 (segment (start 178.325 64.625) (end 177.675 63.975) (width 0.2) (layer "F.Cu") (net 1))
 (segment (start 178.325 66.1125) (end 178.325 64.625) (width 0.2) (layer "F.Cu") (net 1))
 (segment (start 181.764 59.224) (end 184 61.46) (width 0.2) (layer "F.Cu") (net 1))
 (segment (start 176.6375 60.0375) (end 176.6375 60) (width 0.2) (layer "F.Cu") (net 1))
 (segment (start 177.675 63.975) (end 177.675 61.8875) (width 0.2) (layer "F.Cu") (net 1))
 (segment (start 179.9 67.9) (end 180.6375 68.6375) (width 0.2) (layer "F.Cu") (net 3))
 (segment (start 180.6375 68.6375) (end 181.9025 68.6375) (width 0.2) (layer "F.Cu") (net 3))
 (segment (start 177.675 67.925) (end 177 68.6) (width 0.2) (layer "F.Cu") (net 3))
 (segment (start 177 68.6) (end 177 68.707) (width 0.2) (layer "F.Cu") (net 3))
 (segment (start 177.675 66.1125) (end 177.675 67.9) (width 0.2) (layer "F.Cu") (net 3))
 (segment (start 181.9025 68.6375) (end 184 66.54) (width 0.2) (layer "F.Cu") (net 3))
 (segment (start 177.675 67.9) (end 179.9 67.9) (width 0.2) (layer "F.Cu") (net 3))
 (segment (start 177.675 67.9) (end 177.675 67.925) (width 0.2) (layer "F.Cu") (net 3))
 (segment (start 175.7875 66.1125) (end 177.025 66.1125) (width 0.2) (layer "F.Cu") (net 6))
 (segment (start 175.36 66.54) (end 175.7875 66.1125) (width 0.2) (layer "F.Cu") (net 6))
 (segment (start 174 66.54) (end 175.36 66.54) (width 0.2) (layer "F.Cu") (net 6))
 (segment (start 175.7875 61.8875) (end 177.025 61.8875) (width 0.2) (layer "F.Cu") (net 7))
 (segment (start 175.36 61.46) (end 175.7875 61.8875) (width 0.2) (layer "F.Cu") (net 7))
 (segment (start 174 61.46) (end 175.36 61.46) (width 0.2) (layer "F.Cu") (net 7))
 (segment (start 179.0875 61.8875) (end 180.2875 63.0875) (width 0.2) (layer "F.Cu") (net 5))
 (segment (start 178.6 60.8) (end 178.8 60.8) (width 0.2) (layer "F.Cu") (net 5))
 (segment (start 178.325 61.8875) (end 178.325 61.075) (width 0.2) (layer "F.Cu") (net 5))
 (segment (start 178.975 61.8875) (end 179.0875 61.8875) (width 0.2) (layer "F.Cu") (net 5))
 (segment (start 180.2875 63.0875) (end 181 63.0875) (width 0.2) (layer "F.Cu") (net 5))
 (segment (start 178.975 60.975) (end 178.975 61.8875) (width 0.2) (layer "F.Cu") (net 5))
 (segment (start 178.325 61.075) (end 178.6 60.8) (width 0.2) (layer "F.Cu") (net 5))
 (segment (start 178.8 60.8) (end 178.975 60.975) (width 0.2) (layer "F.Cu") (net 5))
 (segment (start 193.878 63.822) (end 206 63.822) (width 0.2) (layer "F.Cu") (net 4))
 (segment (start 181 64.9125) (end 181.3875 65.3) (width 0.2) (layer "F.Cu") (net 4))
 (segment (start 192.4 65.3) (end 193.878 63.822) (width 0.2) (layer "F.Cu") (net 4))
 (segment (start 181.3875 65.3) (end 192.4 65.3) (width 0.2) (layer "F.Cu") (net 4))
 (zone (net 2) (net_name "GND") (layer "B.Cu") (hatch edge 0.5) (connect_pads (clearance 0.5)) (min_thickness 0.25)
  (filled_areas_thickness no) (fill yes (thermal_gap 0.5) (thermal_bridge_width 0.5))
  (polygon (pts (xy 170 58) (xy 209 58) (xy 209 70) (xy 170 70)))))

